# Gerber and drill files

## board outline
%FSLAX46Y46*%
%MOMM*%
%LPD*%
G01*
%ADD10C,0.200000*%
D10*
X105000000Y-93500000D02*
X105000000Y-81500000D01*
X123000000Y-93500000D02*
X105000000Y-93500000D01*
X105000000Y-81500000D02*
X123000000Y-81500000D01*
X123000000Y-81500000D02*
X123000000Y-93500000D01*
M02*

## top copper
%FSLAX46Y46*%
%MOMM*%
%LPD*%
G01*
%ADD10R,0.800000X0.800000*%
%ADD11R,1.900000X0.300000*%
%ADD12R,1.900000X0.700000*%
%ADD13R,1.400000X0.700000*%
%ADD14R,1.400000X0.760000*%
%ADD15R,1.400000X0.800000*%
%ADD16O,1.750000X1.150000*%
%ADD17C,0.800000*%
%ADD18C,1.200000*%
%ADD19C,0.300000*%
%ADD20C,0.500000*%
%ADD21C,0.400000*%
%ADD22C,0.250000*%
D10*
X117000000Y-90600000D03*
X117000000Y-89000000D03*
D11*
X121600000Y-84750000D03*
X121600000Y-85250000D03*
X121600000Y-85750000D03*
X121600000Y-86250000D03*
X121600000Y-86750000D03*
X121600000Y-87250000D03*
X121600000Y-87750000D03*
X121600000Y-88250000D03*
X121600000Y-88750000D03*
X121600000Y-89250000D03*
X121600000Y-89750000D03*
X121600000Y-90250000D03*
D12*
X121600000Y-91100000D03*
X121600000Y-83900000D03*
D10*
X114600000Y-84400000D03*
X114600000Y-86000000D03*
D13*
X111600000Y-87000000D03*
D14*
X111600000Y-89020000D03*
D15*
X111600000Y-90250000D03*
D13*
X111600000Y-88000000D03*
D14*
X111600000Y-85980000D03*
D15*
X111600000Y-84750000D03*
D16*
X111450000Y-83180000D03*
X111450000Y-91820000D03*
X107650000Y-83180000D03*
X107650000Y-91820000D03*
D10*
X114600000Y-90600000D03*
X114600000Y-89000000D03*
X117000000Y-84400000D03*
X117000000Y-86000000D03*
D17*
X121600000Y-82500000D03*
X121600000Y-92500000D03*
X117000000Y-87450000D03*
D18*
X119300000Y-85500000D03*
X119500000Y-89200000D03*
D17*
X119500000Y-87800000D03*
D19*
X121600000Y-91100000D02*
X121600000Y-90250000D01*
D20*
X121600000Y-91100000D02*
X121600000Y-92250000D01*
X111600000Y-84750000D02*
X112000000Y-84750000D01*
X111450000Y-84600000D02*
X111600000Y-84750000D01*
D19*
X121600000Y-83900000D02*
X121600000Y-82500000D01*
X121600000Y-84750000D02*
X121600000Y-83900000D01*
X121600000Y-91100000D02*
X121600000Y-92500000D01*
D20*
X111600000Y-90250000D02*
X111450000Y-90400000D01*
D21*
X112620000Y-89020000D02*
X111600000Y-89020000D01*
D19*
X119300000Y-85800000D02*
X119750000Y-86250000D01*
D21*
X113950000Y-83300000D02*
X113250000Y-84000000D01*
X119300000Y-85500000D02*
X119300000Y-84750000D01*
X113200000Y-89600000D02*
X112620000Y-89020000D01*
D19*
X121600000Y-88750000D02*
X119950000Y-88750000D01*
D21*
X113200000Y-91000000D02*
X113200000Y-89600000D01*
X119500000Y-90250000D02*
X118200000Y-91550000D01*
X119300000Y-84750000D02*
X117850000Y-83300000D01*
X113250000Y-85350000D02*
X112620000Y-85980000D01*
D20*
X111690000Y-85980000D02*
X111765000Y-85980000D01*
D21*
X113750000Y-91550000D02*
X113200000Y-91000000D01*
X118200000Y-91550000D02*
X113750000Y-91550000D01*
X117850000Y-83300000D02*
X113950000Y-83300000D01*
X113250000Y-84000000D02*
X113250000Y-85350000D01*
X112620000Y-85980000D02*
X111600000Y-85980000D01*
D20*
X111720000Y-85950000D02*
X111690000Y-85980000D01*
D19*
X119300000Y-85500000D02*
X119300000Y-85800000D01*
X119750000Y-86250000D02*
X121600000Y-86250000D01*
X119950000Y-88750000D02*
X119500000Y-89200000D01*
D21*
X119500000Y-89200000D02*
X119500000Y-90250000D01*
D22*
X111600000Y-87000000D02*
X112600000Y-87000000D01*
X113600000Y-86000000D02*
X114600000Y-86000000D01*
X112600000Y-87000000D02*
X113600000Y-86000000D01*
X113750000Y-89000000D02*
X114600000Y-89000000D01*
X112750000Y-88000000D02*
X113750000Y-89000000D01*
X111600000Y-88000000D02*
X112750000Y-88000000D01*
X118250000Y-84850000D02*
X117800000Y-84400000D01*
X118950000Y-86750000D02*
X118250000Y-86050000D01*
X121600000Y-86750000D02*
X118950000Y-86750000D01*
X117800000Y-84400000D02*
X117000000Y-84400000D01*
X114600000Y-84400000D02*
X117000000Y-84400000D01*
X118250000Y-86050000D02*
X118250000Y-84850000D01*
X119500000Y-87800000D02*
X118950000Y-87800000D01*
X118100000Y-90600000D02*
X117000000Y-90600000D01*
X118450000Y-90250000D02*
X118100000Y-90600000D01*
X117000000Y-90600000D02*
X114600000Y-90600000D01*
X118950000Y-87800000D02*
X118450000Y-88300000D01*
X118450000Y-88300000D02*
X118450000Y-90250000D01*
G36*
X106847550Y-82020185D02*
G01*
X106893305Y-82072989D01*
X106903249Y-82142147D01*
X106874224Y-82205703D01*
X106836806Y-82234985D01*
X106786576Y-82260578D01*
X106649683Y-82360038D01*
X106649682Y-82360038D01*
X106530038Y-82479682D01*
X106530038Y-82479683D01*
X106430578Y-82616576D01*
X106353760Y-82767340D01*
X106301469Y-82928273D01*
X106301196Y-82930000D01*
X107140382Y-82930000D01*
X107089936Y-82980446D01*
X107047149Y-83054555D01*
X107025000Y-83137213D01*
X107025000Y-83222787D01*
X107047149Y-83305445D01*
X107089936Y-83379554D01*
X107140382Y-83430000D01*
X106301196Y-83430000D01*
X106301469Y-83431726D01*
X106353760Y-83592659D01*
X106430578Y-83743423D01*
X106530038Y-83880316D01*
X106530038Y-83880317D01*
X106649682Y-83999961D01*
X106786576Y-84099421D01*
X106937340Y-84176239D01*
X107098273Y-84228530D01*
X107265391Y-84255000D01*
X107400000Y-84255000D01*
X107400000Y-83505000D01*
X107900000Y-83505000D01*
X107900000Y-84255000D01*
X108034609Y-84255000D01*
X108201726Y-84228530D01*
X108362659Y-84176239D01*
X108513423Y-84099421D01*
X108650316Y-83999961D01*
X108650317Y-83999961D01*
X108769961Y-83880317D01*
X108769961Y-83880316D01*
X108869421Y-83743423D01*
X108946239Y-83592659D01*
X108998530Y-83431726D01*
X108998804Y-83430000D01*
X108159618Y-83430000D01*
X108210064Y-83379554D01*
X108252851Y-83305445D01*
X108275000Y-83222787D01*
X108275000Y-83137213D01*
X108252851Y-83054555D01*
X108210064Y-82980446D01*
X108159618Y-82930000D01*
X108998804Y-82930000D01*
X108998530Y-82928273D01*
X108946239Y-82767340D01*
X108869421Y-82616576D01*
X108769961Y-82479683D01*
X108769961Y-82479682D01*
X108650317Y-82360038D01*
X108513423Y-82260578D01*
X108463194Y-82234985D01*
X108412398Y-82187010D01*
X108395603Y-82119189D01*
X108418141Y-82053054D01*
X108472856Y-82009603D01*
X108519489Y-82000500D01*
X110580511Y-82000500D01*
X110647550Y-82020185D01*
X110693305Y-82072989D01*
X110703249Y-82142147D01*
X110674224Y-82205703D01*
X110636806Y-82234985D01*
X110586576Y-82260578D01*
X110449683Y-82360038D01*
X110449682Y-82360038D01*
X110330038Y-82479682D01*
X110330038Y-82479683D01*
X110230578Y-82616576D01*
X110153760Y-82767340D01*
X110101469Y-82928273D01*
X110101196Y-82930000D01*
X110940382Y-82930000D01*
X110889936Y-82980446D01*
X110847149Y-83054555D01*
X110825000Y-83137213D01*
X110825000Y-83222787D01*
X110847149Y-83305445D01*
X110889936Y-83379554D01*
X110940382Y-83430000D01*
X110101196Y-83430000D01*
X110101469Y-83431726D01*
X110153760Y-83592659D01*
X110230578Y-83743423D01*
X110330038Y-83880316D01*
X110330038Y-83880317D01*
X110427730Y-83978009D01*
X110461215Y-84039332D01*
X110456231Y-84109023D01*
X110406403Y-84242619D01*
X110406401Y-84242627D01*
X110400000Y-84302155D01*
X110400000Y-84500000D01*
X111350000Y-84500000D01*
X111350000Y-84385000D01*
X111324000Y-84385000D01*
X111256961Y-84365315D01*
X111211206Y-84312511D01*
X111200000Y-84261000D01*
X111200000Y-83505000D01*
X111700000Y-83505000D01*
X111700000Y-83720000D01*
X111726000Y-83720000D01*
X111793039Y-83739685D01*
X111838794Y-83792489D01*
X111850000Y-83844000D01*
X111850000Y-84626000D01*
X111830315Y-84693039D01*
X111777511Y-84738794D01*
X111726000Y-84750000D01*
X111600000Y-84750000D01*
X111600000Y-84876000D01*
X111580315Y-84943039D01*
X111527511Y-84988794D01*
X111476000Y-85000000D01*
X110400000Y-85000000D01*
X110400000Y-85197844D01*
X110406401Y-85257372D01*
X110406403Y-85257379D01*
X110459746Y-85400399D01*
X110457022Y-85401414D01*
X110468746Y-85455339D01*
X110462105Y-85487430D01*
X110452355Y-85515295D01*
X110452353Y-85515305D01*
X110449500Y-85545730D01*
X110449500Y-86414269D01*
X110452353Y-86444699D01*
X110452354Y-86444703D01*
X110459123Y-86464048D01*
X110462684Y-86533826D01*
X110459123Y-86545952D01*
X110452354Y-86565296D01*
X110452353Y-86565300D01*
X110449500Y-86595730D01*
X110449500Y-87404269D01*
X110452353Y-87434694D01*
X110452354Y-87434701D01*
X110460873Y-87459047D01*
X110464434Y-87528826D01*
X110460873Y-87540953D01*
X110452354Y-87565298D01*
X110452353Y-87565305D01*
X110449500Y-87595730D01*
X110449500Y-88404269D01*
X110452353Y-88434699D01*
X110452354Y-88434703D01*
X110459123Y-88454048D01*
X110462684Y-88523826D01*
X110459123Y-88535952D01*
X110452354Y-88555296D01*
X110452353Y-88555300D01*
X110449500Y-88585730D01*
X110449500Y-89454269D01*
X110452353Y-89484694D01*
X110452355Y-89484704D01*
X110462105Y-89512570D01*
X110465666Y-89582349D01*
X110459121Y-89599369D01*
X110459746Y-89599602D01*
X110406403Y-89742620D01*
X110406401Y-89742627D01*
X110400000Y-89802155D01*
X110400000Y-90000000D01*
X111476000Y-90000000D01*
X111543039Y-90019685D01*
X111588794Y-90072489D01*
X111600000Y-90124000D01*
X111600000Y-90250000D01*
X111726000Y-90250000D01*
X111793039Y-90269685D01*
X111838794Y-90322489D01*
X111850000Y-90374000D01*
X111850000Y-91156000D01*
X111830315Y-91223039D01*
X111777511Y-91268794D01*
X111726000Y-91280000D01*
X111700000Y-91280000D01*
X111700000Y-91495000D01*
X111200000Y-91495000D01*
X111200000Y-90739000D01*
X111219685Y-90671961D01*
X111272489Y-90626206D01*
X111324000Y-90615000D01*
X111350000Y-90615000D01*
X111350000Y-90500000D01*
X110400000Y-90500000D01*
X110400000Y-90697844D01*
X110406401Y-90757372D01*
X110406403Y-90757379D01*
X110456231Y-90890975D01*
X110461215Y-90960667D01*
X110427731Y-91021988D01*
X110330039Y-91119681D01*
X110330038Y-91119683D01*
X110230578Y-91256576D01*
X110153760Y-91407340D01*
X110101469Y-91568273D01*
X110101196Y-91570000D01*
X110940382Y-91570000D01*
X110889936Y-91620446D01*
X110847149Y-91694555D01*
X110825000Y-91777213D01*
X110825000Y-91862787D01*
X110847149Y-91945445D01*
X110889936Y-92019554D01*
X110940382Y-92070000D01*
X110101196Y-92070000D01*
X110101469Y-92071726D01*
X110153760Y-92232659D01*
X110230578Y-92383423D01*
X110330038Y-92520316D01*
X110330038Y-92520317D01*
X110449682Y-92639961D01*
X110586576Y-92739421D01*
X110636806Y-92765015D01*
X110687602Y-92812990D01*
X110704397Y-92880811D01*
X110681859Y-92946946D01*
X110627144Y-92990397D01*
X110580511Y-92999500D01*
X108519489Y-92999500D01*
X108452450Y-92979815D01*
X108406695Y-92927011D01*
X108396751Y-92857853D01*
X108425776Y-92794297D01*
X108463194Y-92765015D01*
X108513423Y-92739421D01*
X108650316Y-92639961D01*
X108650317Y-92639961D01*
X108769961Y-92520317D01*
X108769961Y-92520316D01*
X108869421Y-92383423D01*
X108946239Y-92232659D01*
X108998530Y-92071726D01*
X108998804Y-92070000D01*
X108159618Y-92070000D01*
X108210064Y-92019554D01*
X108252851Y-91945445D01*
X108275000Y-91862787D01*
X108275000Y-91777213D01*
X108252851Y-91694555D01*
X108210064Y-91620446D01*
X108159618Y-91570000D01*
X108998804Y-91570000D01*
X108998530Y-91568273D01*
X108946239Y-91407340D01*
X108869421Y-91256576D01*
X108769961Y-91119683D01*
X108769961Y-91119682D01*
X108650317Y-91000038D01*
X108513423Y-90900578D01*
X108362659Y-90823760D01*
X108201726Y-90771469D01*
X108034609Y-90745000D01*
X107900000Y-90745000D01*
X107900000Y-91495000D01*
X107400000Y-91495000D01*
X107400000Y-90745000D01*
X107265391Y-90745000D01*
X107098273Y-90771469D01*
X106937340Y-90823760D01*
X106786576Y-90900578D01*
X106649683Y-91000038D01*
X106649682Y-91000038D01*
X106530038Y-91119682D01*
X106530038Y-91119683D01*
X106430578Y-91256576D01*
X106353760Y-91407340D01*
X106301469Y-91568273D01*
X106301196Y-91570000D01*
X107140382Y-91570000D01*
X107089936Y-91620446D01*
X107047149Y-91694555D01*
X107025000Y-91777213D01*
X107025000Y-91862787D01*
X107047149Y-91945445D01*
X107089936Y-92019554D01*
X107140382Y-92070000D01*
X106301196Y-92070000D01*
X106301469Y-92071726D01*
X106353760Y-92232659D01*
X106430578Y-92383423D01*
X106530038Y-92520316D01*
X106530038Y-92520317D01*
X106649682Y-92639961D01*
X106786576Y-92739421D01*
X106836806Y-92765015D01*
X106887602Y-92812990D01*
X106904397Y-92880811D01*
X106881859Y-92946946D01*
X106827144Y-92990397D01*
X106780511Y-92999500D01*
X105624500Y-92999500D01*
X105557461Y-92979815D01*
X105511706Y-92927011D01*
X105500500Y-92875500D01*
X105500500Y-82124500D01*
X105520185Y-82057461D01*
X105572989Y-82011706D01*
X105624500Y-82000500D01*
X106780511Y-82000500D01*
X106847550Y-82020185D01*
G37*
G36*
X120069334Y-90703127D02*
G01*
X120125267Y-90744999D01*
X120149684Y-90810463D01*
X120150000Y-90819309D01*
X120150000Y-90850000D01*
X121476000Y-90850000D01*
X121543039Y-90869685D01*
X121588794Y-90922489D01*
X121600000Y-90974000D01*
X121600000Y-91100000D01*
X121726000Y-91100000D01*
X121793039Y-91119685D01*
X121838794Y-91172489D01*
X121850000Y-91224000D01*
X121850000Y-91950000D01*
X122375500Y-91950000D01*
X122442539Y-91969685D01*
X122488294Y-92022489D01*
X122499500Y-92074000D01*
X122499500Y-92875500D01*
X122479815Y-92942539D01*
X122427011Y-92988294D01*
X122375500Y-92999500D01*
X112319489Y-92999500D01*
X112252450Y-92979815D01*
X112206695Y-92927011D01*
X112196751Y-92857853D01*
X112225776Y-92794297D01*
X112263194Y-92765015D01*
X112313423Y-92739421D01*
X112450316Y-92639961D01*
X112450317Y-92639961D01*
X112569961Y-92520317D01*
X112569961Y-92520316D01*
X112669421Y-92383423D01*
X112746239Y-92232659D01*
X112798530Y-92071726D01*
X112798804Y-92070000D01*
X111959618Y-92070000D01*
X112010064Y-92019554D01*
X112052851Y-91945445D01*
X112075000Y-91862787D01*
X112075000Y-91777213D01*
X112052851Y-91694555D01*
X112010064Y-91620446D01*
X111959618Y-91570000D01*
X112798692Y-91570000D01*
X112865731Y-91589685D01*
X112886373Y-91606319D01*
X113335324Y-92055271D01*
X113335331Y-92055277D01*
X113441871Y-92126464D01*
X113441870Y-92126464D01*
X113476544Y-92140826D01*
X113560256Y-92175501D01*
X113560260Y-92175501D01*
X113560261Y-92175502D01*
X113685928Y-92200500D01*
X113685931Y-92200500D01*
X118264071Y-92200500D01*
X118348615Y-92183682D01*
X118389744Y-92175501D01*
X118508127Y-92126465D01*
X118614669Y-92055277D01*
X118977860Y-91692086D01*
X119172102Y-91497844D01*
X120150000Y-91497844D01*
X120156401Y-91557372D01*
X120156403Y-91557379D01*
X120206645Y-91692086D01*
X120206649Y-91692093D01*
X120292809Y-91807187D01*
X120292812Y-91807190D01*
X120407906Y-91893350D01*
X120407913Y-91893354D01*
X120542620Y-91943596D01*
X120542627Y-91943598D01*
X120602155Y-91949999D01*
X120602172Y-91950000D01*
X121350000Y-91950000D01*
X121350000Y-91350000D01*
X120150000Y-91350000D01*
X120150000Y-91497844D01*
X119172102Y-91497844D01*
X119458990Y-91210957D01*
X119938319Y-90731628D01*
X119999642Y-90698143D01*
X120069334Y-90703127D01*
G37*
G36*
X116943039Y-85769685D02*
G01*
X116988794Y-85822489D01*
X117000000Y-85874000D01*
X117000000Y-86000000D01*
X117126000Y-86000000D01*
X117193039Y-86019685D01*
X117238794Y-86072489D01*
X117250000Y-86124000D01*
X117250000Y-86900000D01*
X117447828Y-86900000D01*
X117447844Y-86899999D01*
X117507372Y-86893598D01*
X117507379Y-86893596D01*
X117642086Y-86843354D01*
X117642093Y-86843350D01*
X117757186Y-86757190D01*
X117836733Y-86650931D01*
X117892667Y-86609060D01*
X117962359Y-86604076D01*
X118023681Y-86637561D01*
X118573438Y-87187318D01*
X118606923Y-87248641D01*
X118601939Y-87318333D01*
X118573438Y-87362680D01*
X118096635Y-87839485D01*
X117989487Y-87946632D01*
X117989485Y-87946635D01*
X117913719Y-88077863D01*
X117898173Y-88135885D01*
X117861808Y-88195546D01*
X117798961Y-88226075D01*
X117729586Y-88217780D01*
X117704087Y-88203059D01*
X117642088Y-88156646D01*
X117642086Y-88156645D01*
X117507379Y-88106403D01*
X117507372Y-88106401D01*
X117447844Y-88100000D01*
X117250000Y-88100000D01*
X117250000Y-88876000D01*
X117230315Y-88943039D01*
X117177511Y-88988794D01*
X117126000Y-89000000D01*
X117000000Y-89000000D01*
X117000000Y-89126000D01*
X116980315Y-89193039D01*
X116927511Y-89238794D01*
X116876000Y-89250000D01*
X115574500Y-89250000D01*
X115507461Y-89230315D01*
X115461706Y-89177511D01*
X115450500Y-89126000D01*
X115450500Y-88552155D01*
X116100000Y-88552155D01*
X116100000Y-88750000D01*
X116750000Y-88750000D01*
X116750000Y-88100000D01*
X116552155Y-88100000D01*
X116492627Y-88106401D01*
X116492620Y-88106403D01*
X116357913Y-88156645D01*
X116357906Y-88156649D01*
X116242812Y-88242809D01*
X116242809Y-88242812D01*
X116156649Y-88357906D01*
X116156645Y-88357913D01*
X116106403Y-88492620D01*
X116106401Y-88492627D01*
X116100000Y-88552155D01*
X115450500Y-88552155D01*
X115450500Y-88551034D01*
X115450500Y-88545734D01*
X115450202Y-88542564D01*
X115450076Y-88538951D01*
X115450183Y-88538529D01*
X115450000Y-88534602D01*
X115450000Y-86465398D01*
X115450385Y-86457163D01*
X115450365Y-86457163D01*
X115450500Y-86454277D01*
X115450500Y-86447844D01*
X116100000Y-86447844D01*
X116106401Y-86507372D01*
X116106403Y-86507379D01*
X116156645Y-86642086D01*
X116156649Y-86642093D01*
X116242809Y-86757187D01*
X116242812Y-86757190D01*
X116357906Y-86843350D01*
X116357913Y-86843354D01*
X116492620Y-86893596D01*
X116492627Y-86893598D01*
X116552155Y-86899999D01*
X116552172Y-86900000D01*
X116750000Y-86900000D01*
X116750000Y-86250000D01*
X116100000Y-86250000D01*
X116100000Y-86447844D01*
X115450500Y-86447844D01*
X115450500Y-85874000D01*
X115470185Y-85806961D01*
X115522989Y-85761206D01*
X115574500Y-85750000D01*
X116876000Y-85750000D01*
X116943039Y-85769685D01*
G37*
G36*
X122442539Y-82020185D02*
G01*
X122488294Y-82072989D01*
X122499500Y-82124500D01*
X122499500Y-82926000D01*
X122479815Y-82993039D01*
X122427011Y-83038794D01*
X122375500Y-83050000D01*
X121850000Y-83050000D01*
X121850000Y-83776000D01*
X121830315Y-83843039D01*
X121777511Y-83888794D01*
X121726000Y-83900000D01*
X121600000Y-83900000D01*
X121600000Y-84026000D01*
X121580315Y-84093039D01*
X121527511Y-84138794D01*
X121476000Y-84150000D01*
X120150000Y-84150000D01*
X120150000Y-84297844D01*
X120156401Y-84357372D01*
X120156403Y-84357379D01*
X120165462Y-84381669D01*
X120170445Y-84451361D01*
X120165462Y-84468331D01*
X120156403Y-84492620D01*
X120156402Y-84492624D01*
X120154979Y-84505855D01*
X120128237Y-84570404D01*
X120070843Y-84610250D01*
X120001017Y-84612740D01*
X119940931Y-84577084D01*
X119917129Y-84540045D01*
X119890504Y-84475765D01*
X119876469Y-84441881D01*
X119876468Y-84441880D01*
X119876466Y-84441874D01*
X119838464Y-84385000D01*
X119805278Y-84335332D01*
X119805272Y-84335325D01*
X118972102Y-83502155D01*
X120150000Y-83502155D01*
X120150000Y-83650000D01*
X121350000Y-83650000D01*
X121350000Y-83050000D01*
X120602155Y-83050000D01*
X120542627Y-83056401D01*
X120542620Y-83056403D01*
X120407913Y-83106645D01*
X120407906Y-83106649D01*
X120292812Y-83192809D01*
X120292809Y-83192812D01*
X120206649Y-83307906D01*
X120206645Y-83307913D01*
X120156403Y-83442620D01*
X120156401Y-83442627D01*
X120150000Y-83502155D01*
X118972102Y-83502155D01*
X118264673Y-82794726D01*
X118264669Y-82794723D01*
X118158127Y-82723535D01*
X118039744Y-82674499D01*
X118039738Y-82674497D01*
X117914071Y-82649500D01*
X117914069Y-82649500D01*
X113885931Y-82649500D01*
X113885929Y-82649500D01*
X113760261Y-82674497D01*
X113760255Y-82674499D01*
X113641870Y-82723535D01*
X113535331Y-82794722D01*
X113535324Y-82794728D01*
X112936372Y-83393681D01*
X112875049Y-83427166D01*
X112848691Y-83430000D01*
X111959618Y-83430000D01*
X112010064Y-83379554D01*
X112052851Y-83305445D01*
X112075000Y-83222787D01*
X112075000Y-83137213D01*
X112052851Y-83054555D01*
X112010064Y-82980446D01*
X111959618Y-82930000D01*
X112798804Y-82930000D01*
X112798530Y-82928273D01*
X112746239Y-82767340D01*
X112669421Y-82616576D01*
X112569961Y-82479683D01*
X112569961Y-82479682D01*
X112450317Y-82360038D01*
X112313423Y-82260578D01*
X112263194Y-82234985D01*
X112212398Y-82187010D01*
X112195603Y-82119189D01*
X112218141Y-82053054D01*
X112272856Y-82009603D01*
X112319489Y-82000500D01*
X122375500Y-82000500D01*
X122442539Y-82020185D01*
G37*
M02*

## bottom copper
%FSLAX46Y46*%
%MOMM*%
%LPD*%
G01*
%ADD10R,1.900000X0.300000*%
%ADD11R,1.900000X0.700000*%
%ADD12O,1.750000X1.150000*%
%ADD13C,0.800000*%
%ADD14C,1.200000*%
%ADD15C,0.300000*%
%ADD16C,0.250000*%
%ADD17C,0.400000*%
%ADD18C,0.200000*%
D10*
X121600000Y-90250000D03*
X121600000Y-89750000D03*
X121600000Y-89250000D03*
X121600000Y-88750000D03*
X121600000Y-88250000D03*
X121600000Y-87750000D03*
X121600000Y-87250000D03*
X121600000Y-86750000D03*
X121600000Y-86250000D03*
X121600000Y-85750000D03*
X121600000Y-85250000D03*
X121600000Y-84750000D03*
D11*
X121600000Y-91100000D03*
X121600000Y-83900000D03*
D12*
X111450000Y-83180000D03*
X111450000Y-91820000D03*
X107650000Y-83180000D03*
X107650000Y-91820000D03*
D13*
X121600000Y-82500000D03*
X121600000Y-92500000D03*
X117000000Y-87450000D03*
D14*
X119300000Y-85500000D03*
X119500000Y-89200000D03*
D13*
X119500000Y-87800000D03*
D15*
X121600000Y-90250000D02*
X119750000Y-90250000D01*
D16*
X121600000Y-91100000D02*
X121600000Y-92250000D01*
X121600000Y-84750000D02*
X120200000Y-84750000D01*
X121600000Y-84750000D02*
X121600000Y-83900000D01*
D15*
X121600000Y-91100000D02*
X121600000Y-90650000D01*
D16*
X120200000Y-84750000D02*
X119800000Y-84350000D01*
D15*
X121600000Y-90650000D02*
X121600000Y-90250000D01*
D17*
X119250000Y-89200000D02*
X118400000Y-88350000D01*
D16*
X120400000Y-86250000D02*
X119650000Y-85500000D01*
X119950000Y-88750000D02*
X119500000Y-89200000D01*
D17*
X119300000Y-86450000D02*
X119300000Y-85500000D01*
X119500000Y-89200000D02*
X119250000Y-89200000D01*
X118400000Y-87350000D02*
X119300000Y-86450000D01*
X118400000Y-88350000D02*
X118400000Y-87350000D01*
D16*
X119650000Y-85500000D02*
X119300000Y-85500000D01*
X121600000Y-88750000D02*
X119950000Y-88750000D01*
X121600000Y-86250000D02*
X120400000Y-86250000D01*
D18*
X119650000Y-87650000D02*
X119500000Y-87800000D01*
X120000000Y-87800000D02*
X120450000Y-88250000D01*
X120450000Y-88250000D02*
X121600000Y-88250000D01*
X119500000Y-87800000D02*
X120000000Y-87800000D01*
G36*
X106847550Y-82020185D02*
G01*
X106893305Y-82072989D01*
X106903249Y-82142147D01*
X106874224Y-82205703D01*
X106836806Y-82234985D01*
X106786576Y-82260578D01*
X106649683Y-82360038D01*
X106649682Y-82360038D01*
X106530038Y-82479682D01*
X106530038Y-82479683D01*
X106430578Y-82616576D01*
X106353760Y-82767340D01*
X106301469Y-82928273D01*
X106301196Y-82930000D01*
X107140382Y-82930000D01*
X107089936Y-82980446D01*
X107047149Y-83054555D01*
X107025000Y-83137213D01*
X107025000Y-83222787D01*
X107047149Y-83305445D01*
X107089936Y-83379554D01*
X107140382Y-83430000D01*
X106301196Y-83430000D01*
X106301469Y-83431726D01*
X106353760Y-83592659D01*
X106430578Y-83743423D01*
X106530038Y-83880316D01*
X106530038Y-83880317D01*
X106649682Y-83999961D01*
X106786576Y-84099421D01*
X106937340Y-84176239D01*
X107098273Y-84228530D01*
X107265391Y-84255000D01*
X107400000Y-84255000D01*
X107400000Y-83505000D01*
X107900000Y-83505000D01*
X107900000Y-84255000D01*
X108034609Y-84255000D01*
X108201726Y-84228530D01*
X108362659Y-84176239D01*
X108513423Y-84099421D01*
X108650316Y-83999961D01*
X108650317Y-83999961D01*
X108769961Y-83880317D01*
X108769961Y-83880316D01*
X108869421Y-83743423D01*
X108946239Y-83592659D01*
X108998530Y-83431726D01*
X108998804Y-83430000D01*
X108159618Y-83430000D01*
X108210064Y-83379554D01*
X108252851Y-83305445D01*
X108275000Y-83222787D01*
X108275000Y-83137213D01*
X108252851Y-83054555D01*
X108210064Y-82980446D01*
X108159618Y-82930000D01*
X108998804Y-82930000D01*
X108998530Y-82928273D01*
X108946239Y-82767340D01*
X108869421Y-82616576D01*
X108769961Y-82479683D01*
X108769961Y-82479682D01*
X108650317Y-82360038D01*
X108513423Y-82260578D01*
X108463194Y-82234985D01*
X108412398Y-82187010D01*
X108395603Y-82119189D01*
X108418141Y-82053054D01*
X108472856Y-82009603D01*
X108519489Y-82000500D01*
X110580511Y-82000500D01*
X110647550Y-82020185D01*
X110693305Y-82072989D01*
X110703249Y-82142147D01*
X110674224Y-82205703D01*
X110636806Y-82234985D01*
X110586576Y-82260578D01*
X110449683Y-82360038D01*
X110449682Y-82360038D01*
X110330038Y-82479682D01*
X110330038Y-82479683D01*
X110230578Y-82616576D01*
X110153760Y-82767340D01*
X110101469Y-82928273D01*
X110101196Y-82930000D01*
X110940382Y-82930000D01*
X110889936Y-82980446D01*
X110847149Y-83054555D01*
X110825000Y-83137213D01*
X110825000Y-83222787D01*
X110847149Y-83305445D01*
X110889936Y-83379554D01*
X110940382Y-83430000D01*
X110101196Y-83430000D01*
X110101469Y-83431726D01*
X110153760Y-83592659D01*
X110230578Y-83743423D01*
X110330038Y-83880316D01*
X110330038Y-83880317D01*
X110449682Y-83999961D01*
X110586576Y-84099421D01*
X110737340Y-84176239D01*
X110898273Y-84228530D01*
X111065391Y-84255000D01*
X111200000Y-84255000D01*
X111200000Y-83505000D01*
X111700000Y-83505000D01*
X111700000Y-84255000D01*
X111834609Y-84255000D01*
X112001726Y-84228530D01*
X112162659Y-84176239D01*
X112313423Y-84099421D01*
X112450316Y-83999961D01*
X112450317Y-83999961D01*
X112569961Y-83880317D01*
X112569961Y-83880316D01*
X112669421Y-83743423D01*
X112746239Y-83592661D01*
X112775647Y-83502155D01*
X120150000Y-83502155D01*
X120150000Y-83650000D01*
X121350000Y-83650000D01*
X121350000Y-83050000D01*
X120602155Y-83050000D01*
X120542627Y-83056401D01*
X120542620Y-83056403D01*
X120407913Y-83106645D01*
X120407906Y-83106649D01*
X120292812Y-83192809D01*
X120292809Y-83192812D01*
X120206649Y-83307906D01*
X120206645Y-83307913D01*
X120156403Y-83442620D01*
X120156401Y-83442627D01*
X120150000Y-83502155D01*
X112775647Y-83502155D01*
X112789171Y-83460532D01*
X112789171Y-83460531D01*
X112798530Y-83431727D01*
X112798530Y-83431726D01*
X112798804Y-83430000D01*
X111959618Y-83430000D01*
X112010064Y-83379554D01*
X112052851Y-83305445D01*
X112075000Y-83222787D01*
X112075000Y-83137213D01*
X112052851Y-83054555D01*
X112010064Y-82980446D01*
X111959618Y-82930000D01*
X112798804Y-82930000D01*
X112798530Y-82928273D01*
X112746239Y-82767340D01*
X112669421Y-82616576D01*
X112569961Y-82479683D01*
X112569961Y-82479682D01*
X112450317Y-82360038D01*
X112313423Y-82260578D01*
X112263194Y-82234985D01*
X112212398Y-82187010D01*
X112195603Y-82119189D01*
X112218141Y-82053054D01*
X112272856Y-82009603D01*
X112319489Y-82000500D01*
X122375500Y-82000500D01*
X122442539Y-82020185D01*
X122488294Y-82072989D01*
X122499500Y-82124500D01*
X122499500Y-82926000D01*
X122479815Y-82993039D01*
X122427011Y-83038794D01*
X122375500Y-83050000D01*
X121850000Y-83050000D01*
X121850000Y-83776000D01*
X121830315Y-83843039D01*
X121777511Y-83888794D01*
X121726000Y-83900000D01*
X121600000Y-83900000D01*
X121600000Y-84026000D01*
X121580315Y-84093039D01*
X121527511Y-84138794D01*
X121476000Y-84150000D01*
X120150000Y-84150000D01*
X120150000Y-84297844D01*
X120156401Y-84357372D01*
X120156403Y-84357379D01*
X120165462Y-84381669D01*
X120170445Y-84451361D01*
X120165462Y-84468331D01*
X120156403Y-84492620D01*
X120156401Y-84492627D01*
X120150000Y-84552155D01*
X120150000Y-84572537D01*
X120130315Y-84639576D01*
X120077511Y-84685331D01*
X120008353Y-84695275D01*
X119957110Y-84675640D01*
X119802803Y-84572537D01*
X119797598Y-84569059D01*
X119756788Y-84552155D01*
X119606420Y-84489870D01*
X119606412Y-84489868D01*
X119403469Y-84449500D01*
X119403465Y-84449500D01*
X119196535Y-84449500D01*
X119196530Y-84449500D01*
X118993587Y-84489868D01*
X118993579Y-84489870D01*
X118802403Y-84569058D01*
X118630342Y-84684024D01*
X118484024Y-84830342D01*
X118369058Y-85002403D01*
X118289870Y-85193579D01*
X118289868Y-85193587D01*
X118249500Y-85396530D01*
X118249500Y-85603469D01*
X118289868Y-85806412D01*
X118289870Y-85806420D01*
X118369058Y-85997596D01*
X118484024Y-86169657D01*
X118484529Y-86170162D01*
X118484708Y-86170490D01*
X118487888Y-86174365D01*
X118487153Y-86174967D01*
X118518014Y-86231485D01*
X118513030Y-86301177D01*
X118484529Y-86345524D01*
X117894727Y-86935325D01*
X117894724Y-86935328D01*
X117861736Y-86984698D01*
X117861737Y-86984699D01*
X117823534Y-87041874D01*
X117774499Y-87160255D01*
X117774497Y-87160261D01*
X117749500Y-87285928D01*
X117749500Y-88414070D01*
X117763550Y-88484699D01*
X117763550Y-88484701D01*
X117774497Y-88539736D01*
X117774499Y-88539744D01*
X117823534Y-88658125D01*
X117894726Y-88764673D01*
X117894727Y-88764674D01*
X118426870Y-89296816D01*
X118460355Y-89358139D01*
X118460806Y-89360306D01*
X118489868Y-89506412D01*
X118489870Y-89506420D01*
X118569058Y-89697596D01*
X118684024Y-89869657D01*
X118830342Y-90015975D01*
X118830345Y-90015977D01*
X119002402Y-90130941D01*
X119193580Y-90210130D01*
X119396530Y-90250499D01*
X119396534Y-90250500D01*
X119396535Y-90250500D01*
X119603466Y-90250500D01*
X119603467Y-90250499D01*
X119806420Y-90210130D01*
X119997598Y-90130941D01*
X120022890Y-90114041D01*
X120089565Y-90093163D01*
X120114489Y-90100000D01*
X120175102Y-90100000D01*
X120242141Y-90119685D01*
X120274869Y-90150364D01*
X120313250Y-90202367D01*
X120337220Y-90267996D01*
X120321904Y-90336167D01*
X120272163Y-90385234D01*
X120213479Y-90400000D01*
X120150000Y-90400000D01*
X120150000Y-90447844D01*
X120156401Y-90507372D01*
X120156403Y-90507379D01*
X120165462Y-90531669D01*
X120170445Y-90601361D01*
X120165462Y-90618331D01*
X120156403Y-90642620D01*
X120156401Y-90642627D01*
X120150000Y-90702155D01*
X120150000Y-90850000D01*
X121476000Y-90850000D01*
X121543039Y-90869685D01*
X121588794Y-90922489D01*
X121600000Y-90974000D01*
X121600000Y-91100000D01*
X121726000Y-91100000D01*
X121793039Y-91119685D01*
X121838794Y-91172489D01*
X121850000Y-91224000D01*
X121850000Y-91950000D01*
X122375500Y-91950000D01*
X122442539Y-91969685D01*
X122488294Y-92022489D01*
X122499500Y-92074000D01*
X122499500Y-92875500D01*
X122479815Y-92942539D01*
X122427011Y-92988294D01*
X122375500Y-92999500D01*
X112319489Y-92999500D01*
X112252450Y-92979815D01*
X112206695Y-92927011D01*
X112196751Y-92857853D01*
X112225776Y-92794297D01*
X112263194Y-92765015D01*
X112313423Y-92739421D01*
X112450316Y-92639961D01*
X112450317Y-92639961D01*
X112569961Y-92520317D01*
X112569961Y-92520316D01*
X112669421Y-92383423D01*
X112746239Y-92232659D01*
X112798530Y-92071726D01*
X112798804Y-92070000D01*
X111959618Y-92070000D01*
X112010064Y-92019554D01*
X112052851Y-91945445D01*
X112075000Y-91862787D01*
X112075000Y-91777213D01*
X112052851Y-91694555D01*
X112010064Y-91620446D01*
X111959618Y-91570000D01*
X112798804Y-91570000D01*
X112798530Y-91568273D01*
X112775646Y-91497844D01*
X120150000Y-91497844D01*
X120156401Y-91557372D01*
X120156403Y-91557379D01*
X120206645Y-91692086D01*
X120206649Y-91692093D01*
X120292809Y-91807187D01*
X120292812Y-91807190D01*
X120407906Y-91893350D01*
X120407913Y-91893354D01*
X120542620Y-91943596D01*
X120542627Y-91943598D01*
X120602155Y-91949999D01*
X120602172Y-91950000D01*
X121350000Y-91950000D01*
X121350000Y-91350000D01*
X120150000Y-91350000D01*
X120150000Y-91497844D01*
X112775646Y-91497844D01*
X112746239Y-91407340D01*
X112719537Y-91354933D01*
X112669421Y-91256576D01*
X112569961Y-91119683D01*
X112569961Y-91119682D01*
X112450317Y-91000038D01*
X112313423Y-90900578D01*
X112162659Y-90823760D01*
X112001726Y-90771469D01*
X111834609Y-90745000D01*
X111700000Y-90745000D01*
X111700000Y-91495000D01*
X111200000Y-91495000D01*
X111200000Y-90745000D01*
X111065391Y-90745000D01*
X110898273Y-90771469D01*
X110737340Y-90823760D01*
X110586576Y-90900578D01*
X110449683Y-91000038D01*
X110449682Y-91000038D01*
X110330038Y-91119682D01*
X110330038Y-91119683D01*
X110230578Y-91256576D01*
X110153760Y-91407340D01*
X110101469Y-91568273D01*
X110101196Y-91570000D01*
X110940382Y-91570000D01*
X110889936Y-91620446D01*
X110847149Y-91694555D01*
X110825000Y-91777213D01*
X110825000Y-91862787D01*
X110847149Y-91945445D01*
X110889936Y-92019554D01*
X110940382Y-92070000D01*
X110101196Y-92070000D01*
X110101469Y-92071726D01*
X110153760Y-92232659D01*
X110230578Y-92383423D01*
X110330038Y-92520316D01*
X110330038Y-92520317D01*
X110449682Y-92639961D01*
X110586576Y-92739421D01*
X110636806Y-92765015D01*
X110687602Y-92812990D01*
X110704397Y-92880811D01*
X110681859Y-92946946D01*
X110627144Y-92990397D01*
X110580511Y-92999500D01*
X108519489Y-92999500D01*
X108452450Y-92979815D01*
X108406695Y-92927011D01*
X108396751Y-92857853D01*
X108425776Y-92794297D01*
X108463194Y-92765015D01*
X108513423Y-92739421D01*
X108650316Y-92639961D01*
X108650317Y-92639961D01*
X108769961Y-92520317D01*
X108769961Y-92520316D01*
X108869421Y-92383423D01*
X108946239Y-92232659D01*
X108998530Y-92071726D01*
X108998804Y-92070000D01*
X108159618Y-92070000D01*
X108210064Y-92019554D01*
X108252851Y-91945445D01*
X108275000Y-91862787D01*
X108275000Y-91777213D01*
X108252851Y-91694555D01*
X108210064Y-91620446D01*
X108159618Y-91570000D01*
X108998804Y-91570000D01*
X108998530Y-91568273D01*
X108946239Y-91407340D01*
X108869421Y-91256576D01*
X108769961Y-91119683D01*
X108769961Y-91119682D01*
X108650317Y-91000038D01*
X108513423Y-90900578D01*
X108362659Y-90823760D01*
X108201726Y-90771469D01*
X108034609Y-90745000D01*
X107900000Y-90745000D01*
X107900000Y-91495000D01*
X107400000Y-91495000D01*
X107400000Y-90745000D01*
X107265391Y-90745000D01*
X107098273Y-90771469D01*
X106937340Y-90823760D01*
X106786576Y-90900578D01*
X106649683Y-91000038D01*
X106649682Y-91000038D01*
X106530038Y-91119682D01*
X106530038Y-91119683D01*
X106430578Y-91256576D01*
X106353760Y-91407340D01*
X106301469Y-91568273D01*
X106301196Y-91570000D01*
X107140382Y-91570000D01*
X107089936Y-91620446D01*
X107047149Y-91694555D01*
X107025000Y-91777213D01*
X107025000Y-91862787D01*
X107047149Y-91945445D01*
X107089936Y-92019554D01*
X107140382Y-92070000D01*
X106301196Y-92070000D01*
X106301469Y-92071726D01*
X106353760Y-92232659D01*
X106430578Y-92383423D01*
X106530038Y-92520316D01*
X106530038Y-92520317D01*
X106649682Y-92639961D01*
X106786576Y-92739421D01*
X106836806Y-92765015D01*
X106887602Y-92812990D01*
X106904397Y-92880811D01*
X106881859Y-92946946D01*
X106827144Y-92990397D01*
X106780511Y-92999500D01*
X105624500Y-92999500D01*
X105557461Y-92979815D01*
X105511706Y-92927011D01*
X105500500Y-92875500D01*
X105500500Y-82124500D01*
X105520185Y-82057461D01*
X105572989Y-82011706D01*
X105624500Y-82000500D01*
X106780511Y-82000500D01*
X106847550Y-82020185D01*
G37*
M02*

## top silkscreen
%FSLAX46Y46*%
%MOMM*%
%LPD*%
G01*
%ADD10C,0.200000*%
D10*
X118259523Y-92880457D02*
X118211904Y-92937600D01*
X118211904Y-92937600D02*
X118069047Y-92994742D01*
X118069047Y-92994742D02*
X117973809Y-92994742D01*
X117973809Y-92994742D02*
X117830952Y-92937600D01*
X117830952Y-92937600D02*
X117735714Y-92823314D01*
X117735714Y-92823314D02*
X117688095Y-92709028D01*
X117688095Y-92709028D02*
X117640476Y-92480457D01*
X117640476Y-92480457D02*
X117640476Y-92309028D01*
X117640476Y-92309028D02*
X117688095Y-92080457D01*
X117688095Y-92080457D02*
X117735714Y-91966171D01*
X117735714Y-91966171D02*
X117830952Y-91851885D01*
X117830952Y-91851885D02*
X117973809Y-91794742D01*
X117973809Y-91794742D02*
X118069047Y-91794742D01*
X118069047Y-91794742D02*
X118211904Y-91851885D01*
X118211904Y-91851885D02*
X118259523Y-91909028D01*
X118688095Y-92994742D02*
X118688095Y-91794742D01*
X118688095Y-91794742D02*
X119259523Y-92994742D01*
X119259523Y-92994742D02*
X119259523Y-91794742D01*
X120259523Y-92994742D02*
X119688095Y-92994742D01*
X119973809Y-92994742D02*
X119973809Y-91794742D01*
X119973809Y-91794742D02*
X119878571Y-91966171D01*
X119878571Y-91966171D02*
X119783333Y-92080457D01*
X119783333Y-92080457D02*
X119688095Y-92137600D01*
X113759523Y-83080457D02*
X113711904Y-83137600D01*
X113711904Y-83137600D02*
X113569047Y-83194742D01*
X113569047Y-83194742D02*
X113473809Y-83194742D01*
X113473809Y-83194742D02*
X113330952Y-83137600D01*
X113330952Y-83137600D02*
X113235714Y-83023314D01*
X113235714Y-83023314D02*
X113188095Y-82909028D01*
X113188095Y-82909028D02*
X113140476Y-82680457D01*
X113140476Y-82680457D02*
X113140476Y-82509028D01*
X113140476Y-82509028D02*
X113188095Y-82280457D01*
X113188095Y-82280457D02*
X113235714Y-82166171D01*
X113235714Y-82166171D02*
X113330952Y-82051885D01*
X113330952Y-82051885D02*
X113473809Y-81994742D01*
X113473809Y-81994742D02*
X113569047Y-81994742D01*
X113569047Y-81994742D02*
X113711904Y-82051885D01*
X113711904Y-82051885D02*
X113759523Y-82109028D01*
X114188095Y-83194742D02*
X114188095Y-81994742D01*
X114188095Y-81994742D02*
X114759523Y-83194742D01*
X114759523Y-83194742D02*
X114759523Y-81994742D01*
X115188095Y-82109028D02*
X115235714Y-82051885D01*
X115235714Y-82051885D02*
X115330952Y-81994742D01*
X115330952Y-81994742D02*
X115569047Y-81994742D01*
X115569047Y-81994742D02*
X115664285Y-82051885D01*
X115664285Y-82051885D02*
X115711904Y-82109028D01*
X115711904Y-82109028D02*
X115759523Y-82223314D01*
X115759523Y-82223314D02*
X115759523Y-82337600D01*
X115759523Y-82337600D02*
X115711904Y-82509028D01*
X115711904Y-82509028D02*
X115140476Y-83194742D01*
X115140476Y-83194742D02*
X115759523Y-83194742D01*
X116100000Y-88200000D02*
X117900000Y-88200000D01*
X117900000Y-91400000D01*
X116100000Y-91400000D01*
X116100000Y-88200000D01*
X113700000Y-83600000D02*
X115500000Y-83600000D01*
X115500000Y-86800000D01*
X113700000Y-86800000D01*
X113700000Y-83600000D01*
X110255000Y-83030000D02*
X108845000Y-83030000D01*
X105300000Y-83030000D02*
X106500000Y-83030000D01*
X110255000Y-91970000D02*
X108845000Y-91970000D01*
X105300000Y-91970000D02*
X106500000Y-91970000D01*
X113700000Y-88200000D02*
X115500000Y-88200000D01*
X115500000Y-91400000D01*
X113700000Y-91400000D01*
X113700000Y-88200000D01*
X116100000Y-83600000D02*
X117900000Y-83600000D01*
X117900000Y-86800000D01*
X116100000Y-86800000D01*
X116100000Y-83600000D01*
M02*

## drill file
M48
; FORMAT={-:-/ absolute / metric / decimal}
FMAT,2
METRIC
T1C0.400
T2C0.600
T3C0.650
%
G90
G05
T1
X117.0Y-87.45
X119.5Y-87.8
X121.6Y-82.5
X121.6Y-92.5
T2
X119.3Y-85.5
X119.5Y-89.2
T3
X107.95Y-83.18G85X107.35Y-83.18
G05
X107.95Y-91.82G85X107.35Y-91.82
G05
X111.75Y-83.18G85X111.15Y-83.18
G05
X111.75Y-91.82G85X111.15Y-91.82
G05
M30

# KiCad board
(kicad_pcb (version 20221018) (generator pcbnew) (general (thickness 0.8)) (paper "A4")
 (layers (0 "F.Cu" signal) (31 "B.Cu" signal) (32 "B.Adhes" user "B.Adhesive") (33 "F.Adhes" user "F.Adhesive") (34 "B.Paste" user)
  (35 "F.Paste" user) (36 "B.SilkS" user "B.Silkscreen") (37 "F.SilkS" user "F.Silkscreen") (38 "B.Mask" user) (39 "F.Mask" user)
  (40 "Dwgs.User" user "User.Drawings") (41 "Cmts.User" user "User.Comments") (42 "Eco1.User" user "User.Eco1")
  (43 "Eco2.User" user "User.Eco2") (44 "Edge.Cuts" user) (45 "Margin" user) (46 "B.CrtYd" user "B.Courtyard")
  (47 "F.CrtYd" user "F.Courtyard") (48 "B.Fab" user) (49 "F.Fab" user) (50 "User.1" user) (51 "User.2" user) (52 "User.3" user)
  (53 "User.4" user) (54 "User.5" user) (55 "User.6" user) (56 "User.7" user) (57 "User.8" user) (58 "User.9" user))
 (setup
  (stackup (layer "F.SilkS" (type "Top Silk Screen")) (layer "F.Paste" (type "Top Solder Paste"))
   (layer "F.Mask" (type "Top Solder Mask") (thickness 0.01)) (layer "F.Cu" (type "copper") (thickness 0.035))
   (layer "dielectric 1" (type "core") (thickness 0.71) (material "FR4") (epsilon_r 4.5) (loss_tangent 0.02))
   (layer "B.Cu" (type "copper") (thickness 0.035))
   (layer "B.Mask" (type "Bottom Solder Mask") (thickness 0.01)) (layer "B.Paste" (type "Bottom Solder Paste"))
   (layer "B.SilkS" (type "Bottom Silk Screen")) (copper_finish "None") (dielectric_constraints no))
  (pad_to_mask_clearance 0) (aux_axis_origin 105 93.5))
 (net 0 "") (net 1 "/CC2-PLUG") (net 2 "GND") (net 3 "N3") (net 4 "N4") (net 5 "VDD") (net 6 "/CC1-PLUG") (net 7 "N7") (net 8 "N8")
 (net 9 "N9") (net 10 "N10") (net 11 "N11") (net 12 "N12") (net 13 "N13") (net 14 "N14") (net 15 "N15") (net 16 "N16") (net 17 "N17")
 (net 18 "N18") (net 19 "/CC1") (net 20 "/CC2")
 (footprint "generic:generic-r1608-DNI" (layer "F.Cu") (at 117 89.8 90)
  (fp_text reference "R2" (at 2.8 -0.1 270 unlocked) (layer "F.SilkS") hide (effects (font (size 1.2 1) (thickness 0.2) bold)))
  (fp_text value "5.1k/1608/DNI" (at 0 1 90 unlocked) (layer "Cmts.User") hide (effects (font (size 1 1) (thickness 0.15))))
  (fp_rect (start -1.6 0.9) (end 1.6 -0.9) (stroke (width 0.2) (type default)) (fill none) (layer "F.SilkS"))
  (pad "1" smd rect (at -0.8 0 90) (size 0.8 0.8) (layers "F.Cu" "F.Mask") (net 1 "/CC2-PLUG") (solder_mask_margin 0.05)
   (thermal_bridge_angle 0))
  (pad "2" smd rect (at 0.8 0 90) (size 0.8 0.8) (layers "F.Cu" "F.Mask") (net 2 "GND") (solder_mask_margin 0.05) (thermal_bridge_angle 0)))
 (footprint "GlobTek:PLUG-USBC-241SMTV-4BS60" (layer "F.Cu") (at 122.9 87.5 90)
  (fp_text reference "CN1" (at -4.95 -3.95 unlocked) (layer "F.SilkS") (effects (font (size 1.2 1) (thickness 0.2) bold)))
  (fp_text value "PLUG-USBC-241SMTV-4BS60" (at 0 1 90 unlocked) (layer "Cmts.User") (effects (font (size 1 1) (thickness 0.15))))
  (pad "A1" smd rect (at 2.75 -1.3 90) (size 0.3 1.9) (layers "F.Cu" "F.Paste" "F.Mask") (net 2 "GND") (solder_mask_margin 0.05)
   (thermal_bridge_angle 0))
  (pad "A2" smd rect (at 2.25 -1.3 90) (size 0.3 1.9) (layers "F.Cu" "F.Paste" "F.Mask") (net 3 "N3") (solder_mask_margin 0.05)
   (thermal_bridge_angle 0))
  (pad "A3" smd rect (at 1.75 -1.3 90) (size 0.3 1.9) (layers "F.Cu" "F.Paste" "F.Mask") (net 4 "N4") (solder_mask_margin 0.05)
   (thermal_bridge_angle 0))
  (pad "A4" smd rect (at 1.25 -1.3 90) (size 0.3 1.9) (layers "F.Cu" "F.Paste" "F.Mask") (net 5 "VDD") (solder_mask_margin 0.05)
   (thermal_bridge_angle 0))
  (pad "A5" smd rect (at 0.75 -1.3 90) (size 0.3 1.9) (layers "F.Cu" "F.Paste" "F.Mask") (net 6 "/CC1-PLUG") (solder_mask_margin 0.05)
   (thermal_bridge_angle 0))
  (pad "A6" smd rect (at 0.25 -1.3 90) (size 0.3 1.9) (layers "F.Cu" "F.Paste" "F.Mask") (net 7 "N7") (solder_mask_margin 0.05)
   (thermal_bridge_angle 0))
  (pad "A7" smd rect (at -0.25 -1.3 90) (size 0.3 1.9) (layers "F.Cu" "F.Paste" "F.Mask") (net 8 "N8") (solder_mask_margin 0.05)
   (thermal_bridge_angle 0))
  (pad "A8" smd rect (at -0.75 -1.3 90) (size 0.3 1.9) (layers "F.Cu" "F.Paste" "F.Mask") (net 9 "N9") (solder_mask_margin 0.05)
   (thermal_bridge_angle 0))
  (pad "A9" smd rect (at -1.25 -1.3 90) (size 0.3 1.9) (layers "F.Cu" "F.Paste" "F.Mask") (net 5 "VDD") (solder_mask_margin 0.05)
   (thermal_bridge_angle 0))
  (pad "A10" smd rect (at -1.75 -1.3 90) (size 0.3 1.9) (layers "F.Cu" "F.Paste" "F.Mask") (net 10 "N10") (solder_mask_margin 0.05)
   (thermal_bridge_angle 0))
  (pad "A11" smd rect (at -2.25 -1.3 90) (size 0.3 1.9) (layers "F.Cu" "F.Paste" "F.Mask") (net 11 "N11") (solder_mask_margin 0.05)
   (thermal_bridge_angle 0))
  (pad "A12" smd rect (at -2.75 -1.3 90) (size 0.3 1.9) (layers "F.Cu" "F.Paste" "F.Mask") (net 2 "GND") (solder_mask_margin 0.05)
   (thermal_bridge_angle 0))
  (pad "B1" smd rect (at -2.75 -1.3 90) (size 0.3 1.9) (layers "B.Cu" "B.Paste" "B.Mask") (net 2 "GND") (solder_mask_margin 0.05)
   (thermal_bridge_angle 0))
  (pad "B2" smd rect (at -2.25 -1.3 90) (size 0.3 1.9) (layers "B.Cu" "B.Paste" "B.Mask") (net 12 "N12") (solder_mask_margin 0.05)
   (thermal_bridge_angle 0))
  (pad "B3" smd rect (at -1.75 -1.3 90) (size 0.3 1.9) (layers "B.Cu" "B.Paste" "B.Mask") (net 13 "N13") (solder_mask_margin 0.05)
   (thermal_bridge_angle 0))
  (pad "B4" smd rect (at -1.25 -1.3 90) (size 0.3 1.9) (layers "B.Cu" "B.Paste" "B.Mask") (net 5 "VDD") (solder_mask_margin 0.05)
   (thermal_bridge_angle 0))
  (pad "B5" smd rect (at -0.75 -1.3 90) (size 0.3 1.9) (layers "B.Cu" "B.Paste" "B.Mask") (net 1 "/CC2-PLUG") (solder_mask_margin 0.05)
   (thermal_bridge_angle 0))
  (pad "B6" smd rect (at -0.25 -1.3 90) (size 0.3 1.9) (layers "B.Cu" "B.Paste" "B.Mask") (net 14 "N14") (solder_mask_margin 0.05)
   (thermal_bridge_angle 0))
  (pad "B7" smd rect (at 0.25 -1.3 90) (size 0.3 1.9) (layers "B.Cu" "B.Paste" "B.Mask") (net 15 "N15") (solder_mask_margin 0.05)
   (thermal_bridge_angle 0))
  (pad "B8" smd rect (at 0.75 -1.3 90) (size 0.3 1.9) (layers "B.Cu" "B.Paste" "B.Mask") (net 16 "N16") (solder_mask_margin 0.05)
   (thermal_bridge_angle 0))
  (pad "B9" smd rect (at 1.25 -1.3 90) (size 0.3 1.9) (layers "B.Cu" "B.Paste" "B.Mask") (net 5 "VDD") (solder_mask_margin 0.05)
   (thermal_bridge_angle 0))
  (pad "B10" smd rect (at 1.75 -1.3 90) (size 0.3 1.9) (layers "B.Cu" "B.Paste" "B.Mask") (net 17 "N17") (solder_mask_margin 0.05)
   (thermal_bridge_angle 0))
  (pad "B11" smd rect (at 2.25 -1.3 90) (size 0.3 1.9) (layers "B.Cu" "B.Paste" "B.Mask") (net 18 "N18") (solder_mask_margin 0.05)
   (thermal_bridge_angle 0))
  (pad "B12" smd rect (at 2.75 -1.3 90) (size 0.3 1.9) (layers "B.Cu" "B.Paste" "B.Mask") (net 2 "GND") (solder_mask_margin 0.05)
   (thermal_bridge_angle 0))
  (pad "SH1" smd rect (at -3.6 -1.3 90) (size 0.7 1.9) (layers "F.Cu" "F.Paste" "F.Mask") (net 2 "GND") (solder_mask_margin 0.05)
   (thermal_bridge_angle 0))
  (pad "SH2" smd rect (at 3.6 -1.3 90) (size 0.7 1.9) (layers "F.Cu" "F.Paste" "F.Mask") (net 2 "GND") (solder_mask_margin 0.05)
   (thermal_bridge_angle 0))
  (pad "SH3" smd rect (at -3.6 -1.3 90) (size 0.7 1.9) (layers "B.Cu" "B.Paste" "B.Mask") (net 2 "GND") (solder_mask_margin 0.05)
   (thermal_bridge_angle 0))
  (pad "SH4" smd rect (at 3.6 -1.3 90) (size 0.7 1.9) (layers "B.Cu" "B.Paste" "B.Mask") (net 2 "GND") (solder_mask_margin 0.05)
   (thermal_bridge_angle 0)))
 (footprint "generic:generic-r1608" (layer "F.Cu") (at 114.6 85.2 -90)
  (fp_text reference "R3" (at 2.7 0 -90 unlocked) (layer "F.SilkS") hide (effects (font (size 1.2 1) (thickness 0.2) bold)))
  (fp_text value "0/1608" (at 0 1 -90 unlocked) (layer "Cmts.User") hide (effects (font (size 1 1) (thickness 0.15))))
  (fp_rect (start -1.6 0.9) (end 1.6 -0.9) (stroke (width 0.2) (type default)) (fill none) (layer "F.SilkS"))
  (pad "1" smd rect (at -0.8 0 270) (size 0.8 0.8) (layers "F.Cu" "F.Paste" "F.Mask") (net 6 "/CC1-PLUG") (solder_mask_margin 0.05)
   (thermal_bridge_angle 0))
  (pad "2" smd rect (at 0.8 0 270) (size 0.8 0.8) (layers "F.Cu" "F.Paste" "F.Mask") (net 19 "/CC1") (solder_mask_margin 0.05)
   (thermal_bridge_angle 0)))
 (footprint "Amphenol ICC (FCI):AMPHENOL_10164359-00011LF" (layer "F.Cu") (at 108.5 87.5 -90)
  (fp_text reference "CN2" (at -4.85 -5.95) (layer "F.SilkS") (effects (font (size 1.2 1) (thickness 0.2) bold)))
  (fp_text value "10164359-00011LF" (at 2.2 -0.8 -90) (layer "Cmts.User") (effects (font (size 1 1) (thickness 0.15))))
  (fp_line (start -4.47 -1.755) (end -4.47 -0.345) (stroke (width 0.2) (type solid)) (layer "F.SilkS"))
  (fp_line (start -4.47 3.2) (end -4.47 2) (stroke (width 0.2) (type solid)) (layer "F.SilkS"))
  (fp_line (start 4.47 -1.755) (end 4.47 -0.345) (stroke (width 0.2) (type solid)) (layer "F.SilkS"))
  (fp_line (start 4.47 3.2) (end 4.47 2) (stroke (width 0.2) (type solid)) (layer "F.SilkS"))
  (pad "A5" smd rect (at -0.5 -3.1 270) (size 0.7 1.4) (layers "F.Cu" "F.Paste" "F.Mask") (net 19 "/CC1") (solder_mask_margin 0.05))
  (pad "A9" smd rect (at 1.52 -3.1 270) (size 0.76 1.4) (layers "F.Cu" "F.Paste" "F.Mask") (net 5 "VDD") (solder_mask_margin 0.05))
  (pad "A12" smd rect (at 2.75 -3.1 270) (size 0.8 1.4) (layers "F.Cu" "F.Paste" "F.Mask") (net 2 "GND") (solder_mask_margin 0.05))
  (pad "B5" smd rect (at 0.5 -3.1 270) (size 0.7 1.4) (layers "F.Cu" "F.Paste" "F.Mask") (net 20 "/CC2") (solder_mask_margin 0.05))
  (pad "B9" smd rect (at -1.52 -3.1 270) (size 0.76 1.4) (layers "F.Cu" "F.Paste" "F.Mask") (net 5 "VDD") (solder_mask_margin 0.05))
  (pad "B12" smd rect (at -2.75 -3.1 270) (size 0.8 1.4) (layers "F.Cu" "F.Paste" "F.Mask") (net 2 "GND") (solder_mask_margin 0.05))
  (pad "SH1" thru_hole oval (at -4.32 -2.95 270) (size 1.15 1.75) (drill oval 0.65 1.25) (layers "*.Cu" "*.Mask") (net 2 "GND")
   (solder_mask_margin 0.102))
  (pad "SH2" thru_hole oval (at 4.32 -2.95 270) (size 1.15 1.75) (drill oval 0.65 1.25) (layers "*.Cu" "*.Mask") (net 2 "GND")
   (solder_mask_margin 0.102))
  (pad "SH3" thru_hole oval (at -4.32 0.85 270) (size 1.15 1.75) (drill oval 0.65 1.25) (layers "*.Cu" "*.Mask") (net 2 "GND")
   (solder_mask_margin 0.102))
  (pad "SH4" thru_hole oval (at 4.32 0.85 270) (size 1.15 1.75) (drill oval 0.65 1.25) (layers "*.Cu" "*.Mask") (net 2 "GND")
   (solder_mask_margin 0.102)))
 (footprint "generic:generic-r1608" (layer "F.Cu") (at 114.6 89.8 90)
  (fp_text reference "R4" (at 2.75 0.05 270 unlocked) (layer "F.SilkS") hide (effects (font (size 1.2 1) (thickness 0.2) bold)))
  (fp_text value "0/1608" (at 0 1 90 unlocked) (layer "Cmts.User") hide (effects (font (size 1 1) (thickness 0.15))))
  (fp_rect (start -1.6 0.9) (end 1.6 -0.9) (stroke (width 0.2) (type default)) (fill none) (layer "F.SilkS"))
  (pad "1" smd rect (at -0.8 0 90) (size 0.8 0.8) (layers "F.Cu" "F.Paste" "F.Mask") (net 1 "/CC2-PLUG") (solder_mask_margin 0.05)
   (thermal_bridge_angle 0))
  (pad "2" smd rect (at 0.8 0 90) (size 0.8 0.8) (layers "F.Cu" "F.Paste" "F.Mask") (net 20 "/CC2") (solder_mask_margin 0.05)
   (thermal_bridge_angle 0)))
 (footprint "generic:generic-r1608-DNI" (layer "F.Cu") (at 117 85.2 -90)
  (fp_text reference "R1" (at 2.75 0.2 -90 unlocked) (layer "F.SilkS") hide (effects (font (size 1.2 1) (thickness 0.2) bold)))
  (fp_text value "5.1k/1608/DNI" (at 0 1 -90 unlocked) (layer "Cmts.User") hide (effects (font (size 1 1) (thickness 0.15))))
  (fp_rect (start -1.6 0.9) (end 1.6 -0.9) (stroke (width 0.2) (type default)) (fill none) (layer "F.SilkS"))
  (pad "1" smd rect (at -0.8 0 270) (size 0.8 0.8) (layers "F.Cu" "F.Mask") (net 6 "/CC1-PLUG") (solder_mask_margin 0.05)
   (thermal_bridge_angle 0))
  (pad "2" smd rect (at 0.8 0 270) (size 0.8 0.8) (layers "F.Cu" "F.Mask") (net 2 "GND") (solder_mask_margin 0.05) (thermal_bridge_angle 0)))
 (gr_line (start 105 93.5) (end 105 81.5) (stroke (width 0.2) (type default)) (layer "Edge.Cuts"))
 (gr_line (start 123 93.5) (end 105 93.5) (stroke (width 0.2) (type default)) (layer "Edge.Cuts"))
 (gr_line (start 105 81.5) (end 123 81.5) (stroke (width 0.2) (type default)) (layer "Edge.Cuts"))
 (gr_line (start 123 81.5) (end 123 93.5) (stroke (width 0.2) (type default)) (layer "Edge.Cuts"))
 (segment (start 121.6 91.1) (end 121.6 90.25) (width 0.3) (layer "F.Cu") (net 2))
 (segment (start 121.6 91.1) (end 121.6 92.25) (width 0.5) (layer "F.Cu") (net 2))
 (segment (start 111.6 84.75) (end 112 84.75) (width 0.5) (layer "F.Cu") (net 2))
 (segment (start 111.45 84.6) (end 111.6 84.75) (width 0.5) (layer "F.Cu") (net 2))
 (segment (start 121.6 83.9) (end 121.6 82.5) (width 0.3) (layer "F.Cu") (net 2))
 (segment (start 121.6 84.75) (end 121.6 83.9) (width 0.3) (layer "F.Cu") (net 2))
 (segment (start 121.6 91.1) (end 121.6 92.5) (width 0.3) (layer "F.Cu") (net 2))
 (segment (start 111.6 90.25) (end 111.45 90.4) (width 0.5) (layer "F.Cu") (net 2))
 (via (at 121.6 82.5) (size 0.8) (drill 0.4) (layers "F.Cu" "B.Cu") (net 2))
 (via (at 121.6 92.5) (size 0.8) (drill 0.4) (layers "F.Cu" "B.Cu") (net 2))
 (via (at 117 87.45) (size 0.8) (drill 0.4) (layers "F.Cu" "B.Cu") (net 2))
 (segment (start 121.6 90.25) (end 119.75 90.25) (width 0.3) (layer "B.Cu") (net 2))
 (segment (start 121.6 91.1) (end 121.6 92.25) (width 0.25) (layer "B.Cu") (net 2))
 (segment (start 121.6 84.75) (end 120.2 84.75) (width 0.25) (layer "B.Cu") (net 2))
 (segment (start 121.6 84.75) (end 121.6 83.9) (width 0.25) (layer "B.Cu") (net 2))
 (segment (start 121.6 91.1) (end 121.6 90.65) (width 0.3) (layer "B.Cu") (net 2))
 (segment (start 120.2 84.75) (end 119.8 84.35) (width 0.25) (layer "B.Cu") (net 2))
 (segment (start 121.6 90.65) (end 121.6 90.25) (width 0.3) (layer "B.Cu") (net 2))
 (segment (start 112.62 89.02) (end 111.6 89.02) (width 0.4) (layer "F.Cu") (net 5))
 (segment (start 119.3 85.8) (end 119.75 86.25) (width 0.3) (layer "F.Cu") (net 5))
 (segment (start 113.95 83.3) (end 113.25 84) (width 0.4) (layer "F.Cu") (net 5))
 (segment (start 119.3 85.5) (end 119.3 84.75) (width 0.4) (layer "F.Cu") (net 5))
 (segment (start 113.2 89.6) (end 112.62 89.02) (width 0.4) (layer "F.Cu") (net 5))
 (segment (start 121.6 88.75) (end 119.95 88.75) (width 0.3) (layer "F.Cu") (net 5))
 (segment (start 113.2 91) (end 113.2 89.6) (width 0.4) (layer "F.Cu") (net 5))
 (segment (start 119.5 90.25) (end 118.2 91.55) (width 0.4) (layer "F.Cu") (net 5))
 (segment (start 119.3 84.75) (end 117.85 83.3) (width 0.4) (layer "F.Cu") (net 5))
 (segment (start 113.25 85.35) (end 112.62 85.98) (width 0.4) (layer "F.Cu") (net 5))
 (segment (start 111.69 85.98) (end 111.765 85.98) (width 0.5) (layer "F.Cu") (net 5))
 (segment (start 113.75 91.55) (end 113.2 91) (width 0.4) (layer "F.Cu") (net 5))
 (segment (start 118.2 91.55) (end 113.75 91.55) (width 0.4) (layer "F.Cu") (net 5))
 (segment (start 117.85 83.3) (end 113.95 83.3) (width 0.4) (layer "F.Cu") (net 5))
 (segment (start 113.25 84) (end 113.25 85.35) (width 0.4) (layer "F.Cu") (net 5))
 (segment (start 112.62 85.98) (end 111.6 85.98) (width 0.4) (layer "F.Cu") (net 5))
 (segment (start 111.72 85.95) (end 111.69 85.98) (width 0.5) (layer "F.Cu") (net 5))
 (segment (start 119.3 85.5) (end 119.3 85.8) (width 0.3) (layer "F.Cu") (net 5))
 (segment (start 119.75 86.25) (end 121.6 86.25) (width 0.3) (layer "F.Cu") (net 5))
 (segment (start 119.95 88.75) (end 119.5 89.2) (width 0.3) (layer "F.Cu") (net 5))
 (segment (start 119.5 89.2) (end 119.5 90.25) (width 0.4) (layer "F.Cu") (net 5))
 (via (at 119.3 85.5) (size 1.2) (drill 0.6) (layers "F.Cu" "B.Cu") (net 5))
 (via (at 119.5 89.2) (size 1.2) (drill 0.6) (layers "F.Cu" "B.Cu") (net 5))
 (segment (start 119.25 89.2) (end 118.4 88.35) (width 0.4) (layer "B.Cu") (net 5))
 (segment (start 120.4 86.25) (end 119.65 85.5) (width 0.25) (layer "B.Cu") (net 5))
 (segment (start 119.95 88.75) (end 119.5 89.2) (width 0.25) (layer "B.Cu") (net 5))
 (segment (start 119.3 86.45) (end 119.3 85.5) (width 0.4) (layer "B.Cu") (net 5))
 (segment (start 119.5 89.2) (end 119.25 89.2) (width 0.4) (layer "B.Cu") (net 5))
 (segment (start 118.4 87.35) (end 119.3 86.45) (width 0.4) (layer "B.Cu") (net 5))
 (segment (start 118.4 88.35) (end 118.4 87.35) (width 0.4) (layer "B.Cu") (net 5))
 (segment (start 119.65 85.5) (end 119.3 85.5) (width 0.25) (layer "B.Cu") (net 5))
 (segment (start 121.6 88.75) (end 119.95 88.75) (width 0.25) (layer "B.Cu") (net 5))
 (segment (start 121.6 86.25) (end 120.4 86.25) (width 0.25) (layer "B.Cu") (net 5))
 (segment (start 111.6 87) (end 112.6 87) (width 0.25) (layer "F.Cu") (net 19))
 (segment (start 113.6 86) (end 114.6 86) (width 0.25) (layer "F.Cu") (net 19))
 (segment (start 112.6 87) (end 113.6 86) (width 0.25) (layer "F.Cu") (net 19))
 (segment (start 113.75 89) (end 114.6 89) (width 0.25) (layer "F.Cu") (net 20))
 (segment (start 112.75 88) (end 113.75 89) (width 0.25) (layer "F.Cu") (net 20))
 (segment (start 111.6 88) (end 112.75 88) (width 0.25) (layer "F.Cu") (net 20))
 (segment (start 118.25 84.85) (end 117.8 84.4) (width 0.25) (layer "F.Cu") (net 6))
 (segment (start 118.95 86.75) (end 118.25 86.05) (width 0.25) (layer "F.Cu") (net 6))
 (segment (start 121.6 86.75) (end 118.95 86.75) (width 0.25) (layer "F.Cu") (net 6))
 (segment (start 117.8 84.4) (end 117 84.4) (width 0.25) (layer "F.Cu") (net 6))
 (segment (start 114.6 84.4) (end 117 84.4) (width 0.25) (layer "F.Cu") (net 6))
 (segment (start 118.25 86.05) (end 118.25 84.85) (width 0.25) (layer "F.Cu") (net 6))
 (segment (start 119.5 87.8) (end 118.95 87.8) (width 0.25) (layer "F.Cu") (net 1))
 (segment (start 118.1 90.6) (end 117 90.6) (width 0.25) (layer "F.Cu") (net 1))
 (segment (start 118.45 90.25) (end 118.1 90.6) (width 0.25) (layer "F.Cu") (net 1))
 (segment (start 117 90.6) (end 114.6 90.6) (width 0.25) (layer "F.Cu") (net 1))
 (segment (start 118.95 87.8) (end 118.45 88.3) (width 0.25) (layer "F.Cu") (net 1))
 (segment (start 118.45 88.3) (end 118.45 90.25) (width 0.25) (layer "F.Cu") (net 1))
 (via (at 119.5 87.8) (size 0.8) (drill 0.4) (layers "F.Cu" "B.Cu") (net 1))
 (segment (start 119.65 87.65) (end 119.5 87.8) (width 0.2) (layer "B.Cu") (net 1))
 (segment (start 120 87.8) (end 120.45 88.25) (width 0.2) (layer "B.Cu") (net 1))
 (segment (start 120.45 88.25) (end 121.6 88.25) (width 0.2) (layer "B.Cu") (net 1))
 (segment (start 119.5 87.8) (end 120 87.8) (width 0.2) (layer "B.Cu") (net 1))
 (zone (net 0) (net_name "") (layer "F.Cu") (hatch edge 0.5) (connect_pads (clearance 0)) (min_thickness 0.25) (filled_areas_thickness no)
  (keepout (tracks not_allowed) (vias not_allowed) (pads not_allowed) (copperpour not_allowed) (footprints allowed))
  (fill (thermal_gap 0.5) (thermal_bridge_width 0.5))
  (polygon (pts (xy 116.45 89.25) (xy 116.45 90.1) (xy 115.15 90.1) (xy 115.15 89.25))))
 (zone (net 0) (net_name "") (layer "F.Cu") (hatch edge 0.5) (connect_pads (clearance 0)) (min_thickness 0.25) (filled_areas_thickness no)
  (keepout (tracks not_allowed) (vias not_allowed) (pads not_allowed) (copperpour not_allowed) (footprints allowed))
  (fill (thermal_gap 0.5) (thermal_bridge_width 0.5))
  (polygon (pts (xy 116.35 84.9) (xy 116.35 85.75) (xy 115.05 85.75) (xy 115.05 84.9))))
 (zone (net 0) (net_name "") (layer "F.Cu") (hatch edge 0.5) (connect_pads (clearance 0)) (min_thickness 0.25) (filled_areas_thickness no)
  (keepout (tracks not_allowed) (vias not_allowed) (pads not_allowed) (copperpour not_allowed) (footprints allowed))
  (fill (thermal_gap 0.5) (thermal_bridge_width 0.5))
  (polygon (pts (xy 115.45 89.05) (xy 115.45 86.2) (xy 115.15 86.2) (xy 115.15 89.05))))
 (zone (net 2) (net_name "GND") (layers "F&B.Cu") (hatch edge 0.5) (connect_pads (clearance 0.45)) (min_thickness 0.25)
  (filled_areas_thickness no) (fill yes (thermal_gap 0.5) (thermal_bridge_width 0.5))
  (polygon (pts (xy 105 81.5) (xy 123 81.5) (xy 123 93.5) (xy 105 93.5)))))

